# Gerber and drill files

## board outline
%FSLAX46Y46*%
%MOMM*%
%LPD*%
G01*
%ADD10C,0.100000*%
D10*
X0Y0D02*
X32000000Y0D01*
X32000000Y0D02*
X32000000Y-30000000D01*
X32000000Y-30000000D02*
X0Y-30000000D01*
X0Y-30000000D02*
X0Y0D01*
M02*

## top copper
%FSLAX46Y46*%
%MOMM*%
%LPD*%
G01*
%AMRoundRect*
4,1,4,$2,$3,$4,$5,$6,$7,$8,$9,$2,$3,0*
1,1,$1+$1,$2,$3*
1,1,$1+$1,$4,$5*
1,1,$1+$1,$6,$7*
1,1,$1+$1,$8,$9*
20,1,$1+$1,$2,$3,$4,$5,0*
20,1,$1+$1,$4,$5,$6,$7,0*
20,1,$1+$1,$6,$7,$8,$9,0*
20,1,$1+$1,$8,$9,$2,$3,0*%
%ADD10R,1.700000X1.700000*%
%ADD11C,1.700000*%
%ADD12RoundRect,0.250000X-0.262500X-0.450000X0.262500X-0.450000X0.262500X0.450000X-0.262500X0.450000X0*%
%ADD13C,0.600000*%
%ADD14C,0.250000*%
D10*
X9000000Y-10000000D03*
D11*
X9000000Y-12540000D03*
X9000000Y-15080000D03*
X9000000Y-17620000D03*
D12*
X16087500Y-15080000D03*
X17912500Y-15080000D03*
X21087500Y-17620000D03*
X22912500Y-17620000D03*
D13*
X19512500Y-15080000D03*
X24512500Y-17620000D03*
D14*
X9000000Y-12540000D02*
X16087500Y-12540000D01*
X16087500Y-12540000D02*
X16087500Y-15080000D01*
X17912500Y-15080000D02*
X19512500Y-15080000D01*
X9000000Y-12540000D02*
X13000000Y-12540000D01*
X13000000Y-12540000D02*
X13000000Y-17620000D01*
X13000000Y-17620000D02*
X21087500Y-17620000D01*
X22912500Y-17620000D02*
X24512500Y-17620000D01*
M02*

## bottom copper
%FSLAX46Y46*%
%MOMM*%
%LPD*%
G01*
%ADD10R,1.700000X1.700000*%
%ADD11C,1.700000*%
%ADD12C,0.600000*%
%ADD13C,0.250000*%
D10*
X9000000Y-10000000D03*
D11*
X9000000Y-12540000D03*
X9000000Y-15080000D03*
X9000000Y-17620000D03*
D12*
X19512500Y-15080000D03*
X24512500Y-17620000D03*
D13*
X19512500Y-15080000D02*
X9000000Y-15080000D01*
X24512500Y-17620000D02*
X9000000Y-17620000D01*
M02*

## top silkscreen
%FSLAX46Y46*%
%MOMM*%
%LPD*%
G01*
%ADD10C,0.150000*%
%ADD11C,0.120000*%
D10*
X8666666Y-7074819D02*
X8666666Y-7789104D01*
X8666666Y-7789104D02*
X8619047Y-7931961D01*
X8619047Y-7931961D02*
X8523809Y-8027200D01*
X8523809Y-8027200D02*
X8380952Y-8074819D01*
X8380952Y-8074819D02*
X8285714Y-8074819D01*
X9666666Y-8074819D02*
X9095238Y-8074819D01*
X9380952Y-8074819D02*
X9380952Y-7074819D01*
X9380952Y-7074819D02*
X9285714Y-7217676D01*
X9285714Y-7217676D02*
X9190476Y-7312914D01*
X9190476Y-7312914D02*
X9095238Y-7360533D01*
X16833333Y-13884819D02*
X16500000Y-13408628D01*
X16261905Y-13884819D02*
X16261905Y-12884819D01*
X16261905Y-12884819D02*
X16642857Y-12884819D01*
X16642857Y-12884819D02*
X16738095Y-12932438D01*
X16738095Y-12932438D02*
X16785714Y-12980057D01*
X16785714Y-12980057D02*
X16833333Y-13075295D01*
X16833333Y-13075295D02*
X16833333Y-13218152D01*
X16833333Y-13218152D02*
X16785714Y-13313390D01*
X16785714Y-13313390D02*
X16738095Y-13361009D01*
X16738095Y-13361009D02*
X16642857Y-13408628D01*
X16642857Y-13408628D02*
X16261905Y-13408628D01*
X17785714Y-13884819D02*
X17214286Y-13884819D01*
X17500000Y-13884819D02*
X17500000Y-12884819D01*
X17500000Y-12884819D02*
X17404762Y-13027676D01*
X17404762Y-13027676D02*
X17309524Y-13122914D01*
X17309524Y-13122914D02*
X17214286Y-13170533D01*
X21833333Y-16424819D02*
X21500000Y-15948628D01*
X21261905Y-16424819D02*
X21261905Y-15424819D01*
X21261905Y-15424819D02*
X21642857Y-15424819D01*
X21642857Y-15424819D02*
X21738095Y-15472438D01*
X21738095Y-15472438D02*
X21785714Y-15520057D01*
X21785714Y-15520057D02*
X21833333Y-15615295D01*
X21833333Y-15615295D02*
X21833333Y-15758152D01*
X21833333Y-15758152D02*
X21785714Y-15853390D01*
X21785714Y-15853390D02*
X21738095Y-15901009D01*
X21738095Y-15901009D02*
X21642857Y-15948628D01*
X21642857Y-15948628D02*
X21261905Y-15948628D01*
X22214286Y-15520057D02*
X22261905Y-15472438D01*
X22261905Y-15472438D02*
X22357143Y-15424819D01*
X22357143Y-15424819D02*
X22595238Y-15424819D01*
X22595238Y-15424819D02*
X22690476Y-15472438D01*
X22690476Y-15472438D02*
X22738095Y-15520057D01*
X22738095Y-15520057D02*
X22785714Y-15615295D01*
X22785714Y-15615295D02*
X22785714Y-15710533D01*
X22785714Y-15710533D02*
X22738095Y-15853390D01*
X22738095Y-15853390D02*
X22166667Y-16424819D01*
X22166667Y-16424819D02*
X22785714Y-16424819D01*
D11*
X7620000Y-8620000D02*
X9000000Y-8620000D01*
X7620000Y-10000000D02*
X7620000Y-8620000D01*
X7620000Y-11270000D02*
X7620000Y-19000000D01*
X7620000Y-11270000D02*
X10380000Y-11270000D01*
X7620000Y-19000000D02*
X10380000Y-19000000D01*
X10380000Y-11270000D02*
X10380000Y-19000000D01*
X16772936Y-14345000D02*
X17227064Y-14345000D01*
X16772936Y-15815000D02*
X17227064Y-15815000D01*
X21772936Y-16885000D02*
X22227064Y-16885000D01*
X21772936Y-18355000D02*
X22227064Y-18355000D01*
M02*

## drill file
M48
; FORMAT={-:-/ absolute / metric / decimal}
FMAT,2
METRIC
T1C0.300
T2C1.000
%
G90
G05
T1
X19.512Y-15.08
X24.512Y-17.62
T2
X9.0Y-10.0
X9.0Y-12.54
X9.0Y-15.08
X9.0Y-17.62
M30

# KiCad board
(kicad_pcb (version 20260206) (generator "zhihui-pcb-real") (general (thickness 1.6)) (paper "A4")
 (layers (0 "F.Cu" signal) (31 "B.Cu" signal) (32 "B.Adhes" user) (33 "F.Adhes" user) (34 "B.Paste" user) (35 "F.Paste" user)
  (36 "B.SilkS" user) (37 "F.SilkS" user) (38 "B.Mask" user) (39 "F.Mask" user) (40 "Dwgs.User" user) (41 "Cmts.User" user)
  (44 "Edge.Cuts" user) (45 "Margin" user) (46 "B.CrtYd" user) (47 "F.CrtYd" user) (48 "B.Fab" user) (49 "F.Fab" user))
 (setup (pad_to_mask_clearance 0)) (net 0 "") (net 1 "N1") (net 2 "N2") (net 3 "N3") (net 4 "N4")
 (gr_line (start 0 0) (end 32 0) (stroke (width 0.1) (type default)) (layer "Edge.Cuts"))
 (gr_line (start 32 0) (end 32 30) (stroke (width 0.1) (type default)) (layer "Edge.Cuts"))
 (gr_line (start 32 30) (end 0 30) (stroke (width 0.1) (type default)) (layer "Edge.Cuts"))
 (gr_line (start 0 30) (end 0 0) (stroke (width 0.1) (type default)) (layer "Edge.Cuts"))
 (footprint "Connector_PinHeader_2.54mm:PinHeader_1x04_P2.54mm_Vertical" (layer "F.Cu")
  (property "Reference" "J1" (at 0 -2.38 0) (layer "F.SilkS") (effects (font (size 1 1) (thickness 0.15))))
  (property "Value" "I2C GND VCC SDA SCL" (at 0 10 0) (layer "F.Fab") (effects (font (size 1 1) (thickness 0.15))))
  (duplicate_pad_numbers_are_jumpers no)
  (fp_line (start -1.38 -1.38) (end 0 -1.38) (stroke (width 0.12) (type solid)) (layer "F.SilkS"))
  (fp_line (start -1.38 0) (end -1.38 -1.38) (stroke (width 0.12) (type solid)) (layer "F.SilkS"))
  (fp_line (start -1.38 1.27) (end -1.38 9) (stroke (width 0.12) (type solid)) (layer "F.SilkS"))
  (fp_line (start -1.38 1.27) (end 1.38 1.27) (stroke (width 0.12) (type solid)) (layer "F.SilkS"))
  (fp_line (start -1.38 9) (end 1.38 9) (stroke (width 0.12) (type solid)) (layer "F.SilkS"))
  (fp_line (start 1.38 1.27) (end 1.38 9) (stroke (width 0.12) (type solid)) (layer "F.SilkS"))
  (pad "1" thru_hole rect (at 0 0) (size 1.7 1.7) (drill 1) (layers "*.Cu" "*.Mask") (remove_unused_layers no) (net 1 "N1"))
  (pad "2" thru_hole circle (at 0 2.54) (size 1.7 1.7) (drill 1) (layers "*.Cu" "*.Mask") (remove_unused_layers no) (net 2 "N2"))
  (pad "3" thru_hole circle (at 0 5.08) (size 1.7 1.7) (drill 1) (layers "*.Cu" "*.Mask") (remove_unused_layers no) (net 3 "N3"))
  (pad "4" thru_hole circle (at 0 7.62) (size 1.7 1.7) (drill 1) (layers "*.Cu" "*.Mask") (remove_unused_layers no) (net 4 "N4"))
  (at 9 10 0))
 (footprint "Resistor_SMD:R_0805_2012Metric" (layer "F.Cu")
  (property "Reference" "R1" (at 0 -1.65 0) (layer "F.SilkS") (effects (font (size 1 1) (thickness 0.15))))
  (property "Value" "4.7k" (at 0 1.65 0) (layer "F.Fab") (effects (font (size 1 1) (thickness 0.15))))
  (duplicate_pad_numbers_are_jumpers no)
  (fp_line (start -0.227064 -0.735) (end 0.227064 -0.735) (stroke (width 0.12) (type solid)) (layer "F.SilkS"))
  (fp_line (start -0.227064 0.735) (end 0.227064 0.735) (stroke (width 0.12) (type solid)) (layer "F.SilkS"))
  (pad "1" smd roundrect (at -0.9125 0) (size 1.025 1.4) (layers "F.Cu" "F.Mask" "F.Paste") (roundrect_rratio 0.243902) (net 2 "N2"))
  (pad "2" smd roundrect (at 0.9125 0) (size 1.025 1.4) (layers "F.Cu" "F.Mask" "F.Paste") (roundrect_rratio 0.243902) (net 3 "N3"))
  (at 17 15.08 0))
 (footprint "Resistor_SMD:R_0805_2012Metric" (layer "F.Cu")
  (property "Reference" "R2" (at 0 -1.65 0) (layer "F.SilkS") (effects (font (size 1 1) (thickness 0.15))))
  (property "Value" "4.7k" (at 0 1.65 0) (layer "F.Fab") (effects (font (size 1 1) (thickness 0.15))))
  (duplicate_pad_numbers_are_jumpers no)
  (fp_line (start -0.227064 -0.735) (end 0.227064 -0.735) (stroke (width 0.12) (type solid)) (layer "F.SilkS"))
  (fp_line (start -0.227064 0.735) (end 0.227064 0.735) (stroke (width 0.12) (type solid)) (layer "F.SilkS"))
  (pad "1" smd roundrect (at -0.9125 0) (size 1.025 1.4) (layers "F.Cu" "F.Mask" "F.Paste") (roundrect_rratio 0.243902) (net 2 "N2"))
  (pad "2" smd roundrect (at 0.9125 0) (size 1.025 1.4) (layers "F.Cu" "F.Mask" "F.Paste") (roundrect_rratio 0.243902) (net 4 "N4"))
  (at 22 17.62 0))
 (segment (start 9 12.54) (end 16.0875 12.54) (width 0.25) (layer "F.Cu") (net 2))
 (segment (start 16.0875 12.54) (end 16.0875 15.08) (width 0.25) (layer "F.Cu") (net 2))
 (segment (start 17.9125 15.08) (end 19.5125 15.08) (width 0.25) (layer "F.Cu") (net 3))
 (segment (start 19.5125 15.08) (end 9 15.08) (width 0.25) (layer "B.Cu") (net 3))
 (segment (start 9 12.54) (end 13 12.54) (width 0.25) (layer "F.Cu") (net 2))
 (segment (start 13 12.54) (end 13 17.62) (width 0.25) (layer "F.Cu") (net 2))
 (segment (start 13 17.62) (end 21.0875 17.62) (width 0.25) (layer "F.Cu") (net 2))
 (segment (start 22.9125 17.62) (end 24.5125 17.62) (width 0.25) (layer "F.Cu") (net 4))
 (segment (start 24.5125 17.62) (end 9 17.62) (width 0.25) (layer "B.Cu") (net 4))
 (via (at 19.5125 15.08) (size 0.6) (drill 0.3) (layers "F.Cu" "B.Cu") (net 3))
 (via (at 24.5125 17.62) (size 0.6) (drill 0.3) (layers "F.Cu" "B.Cu") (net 4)))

